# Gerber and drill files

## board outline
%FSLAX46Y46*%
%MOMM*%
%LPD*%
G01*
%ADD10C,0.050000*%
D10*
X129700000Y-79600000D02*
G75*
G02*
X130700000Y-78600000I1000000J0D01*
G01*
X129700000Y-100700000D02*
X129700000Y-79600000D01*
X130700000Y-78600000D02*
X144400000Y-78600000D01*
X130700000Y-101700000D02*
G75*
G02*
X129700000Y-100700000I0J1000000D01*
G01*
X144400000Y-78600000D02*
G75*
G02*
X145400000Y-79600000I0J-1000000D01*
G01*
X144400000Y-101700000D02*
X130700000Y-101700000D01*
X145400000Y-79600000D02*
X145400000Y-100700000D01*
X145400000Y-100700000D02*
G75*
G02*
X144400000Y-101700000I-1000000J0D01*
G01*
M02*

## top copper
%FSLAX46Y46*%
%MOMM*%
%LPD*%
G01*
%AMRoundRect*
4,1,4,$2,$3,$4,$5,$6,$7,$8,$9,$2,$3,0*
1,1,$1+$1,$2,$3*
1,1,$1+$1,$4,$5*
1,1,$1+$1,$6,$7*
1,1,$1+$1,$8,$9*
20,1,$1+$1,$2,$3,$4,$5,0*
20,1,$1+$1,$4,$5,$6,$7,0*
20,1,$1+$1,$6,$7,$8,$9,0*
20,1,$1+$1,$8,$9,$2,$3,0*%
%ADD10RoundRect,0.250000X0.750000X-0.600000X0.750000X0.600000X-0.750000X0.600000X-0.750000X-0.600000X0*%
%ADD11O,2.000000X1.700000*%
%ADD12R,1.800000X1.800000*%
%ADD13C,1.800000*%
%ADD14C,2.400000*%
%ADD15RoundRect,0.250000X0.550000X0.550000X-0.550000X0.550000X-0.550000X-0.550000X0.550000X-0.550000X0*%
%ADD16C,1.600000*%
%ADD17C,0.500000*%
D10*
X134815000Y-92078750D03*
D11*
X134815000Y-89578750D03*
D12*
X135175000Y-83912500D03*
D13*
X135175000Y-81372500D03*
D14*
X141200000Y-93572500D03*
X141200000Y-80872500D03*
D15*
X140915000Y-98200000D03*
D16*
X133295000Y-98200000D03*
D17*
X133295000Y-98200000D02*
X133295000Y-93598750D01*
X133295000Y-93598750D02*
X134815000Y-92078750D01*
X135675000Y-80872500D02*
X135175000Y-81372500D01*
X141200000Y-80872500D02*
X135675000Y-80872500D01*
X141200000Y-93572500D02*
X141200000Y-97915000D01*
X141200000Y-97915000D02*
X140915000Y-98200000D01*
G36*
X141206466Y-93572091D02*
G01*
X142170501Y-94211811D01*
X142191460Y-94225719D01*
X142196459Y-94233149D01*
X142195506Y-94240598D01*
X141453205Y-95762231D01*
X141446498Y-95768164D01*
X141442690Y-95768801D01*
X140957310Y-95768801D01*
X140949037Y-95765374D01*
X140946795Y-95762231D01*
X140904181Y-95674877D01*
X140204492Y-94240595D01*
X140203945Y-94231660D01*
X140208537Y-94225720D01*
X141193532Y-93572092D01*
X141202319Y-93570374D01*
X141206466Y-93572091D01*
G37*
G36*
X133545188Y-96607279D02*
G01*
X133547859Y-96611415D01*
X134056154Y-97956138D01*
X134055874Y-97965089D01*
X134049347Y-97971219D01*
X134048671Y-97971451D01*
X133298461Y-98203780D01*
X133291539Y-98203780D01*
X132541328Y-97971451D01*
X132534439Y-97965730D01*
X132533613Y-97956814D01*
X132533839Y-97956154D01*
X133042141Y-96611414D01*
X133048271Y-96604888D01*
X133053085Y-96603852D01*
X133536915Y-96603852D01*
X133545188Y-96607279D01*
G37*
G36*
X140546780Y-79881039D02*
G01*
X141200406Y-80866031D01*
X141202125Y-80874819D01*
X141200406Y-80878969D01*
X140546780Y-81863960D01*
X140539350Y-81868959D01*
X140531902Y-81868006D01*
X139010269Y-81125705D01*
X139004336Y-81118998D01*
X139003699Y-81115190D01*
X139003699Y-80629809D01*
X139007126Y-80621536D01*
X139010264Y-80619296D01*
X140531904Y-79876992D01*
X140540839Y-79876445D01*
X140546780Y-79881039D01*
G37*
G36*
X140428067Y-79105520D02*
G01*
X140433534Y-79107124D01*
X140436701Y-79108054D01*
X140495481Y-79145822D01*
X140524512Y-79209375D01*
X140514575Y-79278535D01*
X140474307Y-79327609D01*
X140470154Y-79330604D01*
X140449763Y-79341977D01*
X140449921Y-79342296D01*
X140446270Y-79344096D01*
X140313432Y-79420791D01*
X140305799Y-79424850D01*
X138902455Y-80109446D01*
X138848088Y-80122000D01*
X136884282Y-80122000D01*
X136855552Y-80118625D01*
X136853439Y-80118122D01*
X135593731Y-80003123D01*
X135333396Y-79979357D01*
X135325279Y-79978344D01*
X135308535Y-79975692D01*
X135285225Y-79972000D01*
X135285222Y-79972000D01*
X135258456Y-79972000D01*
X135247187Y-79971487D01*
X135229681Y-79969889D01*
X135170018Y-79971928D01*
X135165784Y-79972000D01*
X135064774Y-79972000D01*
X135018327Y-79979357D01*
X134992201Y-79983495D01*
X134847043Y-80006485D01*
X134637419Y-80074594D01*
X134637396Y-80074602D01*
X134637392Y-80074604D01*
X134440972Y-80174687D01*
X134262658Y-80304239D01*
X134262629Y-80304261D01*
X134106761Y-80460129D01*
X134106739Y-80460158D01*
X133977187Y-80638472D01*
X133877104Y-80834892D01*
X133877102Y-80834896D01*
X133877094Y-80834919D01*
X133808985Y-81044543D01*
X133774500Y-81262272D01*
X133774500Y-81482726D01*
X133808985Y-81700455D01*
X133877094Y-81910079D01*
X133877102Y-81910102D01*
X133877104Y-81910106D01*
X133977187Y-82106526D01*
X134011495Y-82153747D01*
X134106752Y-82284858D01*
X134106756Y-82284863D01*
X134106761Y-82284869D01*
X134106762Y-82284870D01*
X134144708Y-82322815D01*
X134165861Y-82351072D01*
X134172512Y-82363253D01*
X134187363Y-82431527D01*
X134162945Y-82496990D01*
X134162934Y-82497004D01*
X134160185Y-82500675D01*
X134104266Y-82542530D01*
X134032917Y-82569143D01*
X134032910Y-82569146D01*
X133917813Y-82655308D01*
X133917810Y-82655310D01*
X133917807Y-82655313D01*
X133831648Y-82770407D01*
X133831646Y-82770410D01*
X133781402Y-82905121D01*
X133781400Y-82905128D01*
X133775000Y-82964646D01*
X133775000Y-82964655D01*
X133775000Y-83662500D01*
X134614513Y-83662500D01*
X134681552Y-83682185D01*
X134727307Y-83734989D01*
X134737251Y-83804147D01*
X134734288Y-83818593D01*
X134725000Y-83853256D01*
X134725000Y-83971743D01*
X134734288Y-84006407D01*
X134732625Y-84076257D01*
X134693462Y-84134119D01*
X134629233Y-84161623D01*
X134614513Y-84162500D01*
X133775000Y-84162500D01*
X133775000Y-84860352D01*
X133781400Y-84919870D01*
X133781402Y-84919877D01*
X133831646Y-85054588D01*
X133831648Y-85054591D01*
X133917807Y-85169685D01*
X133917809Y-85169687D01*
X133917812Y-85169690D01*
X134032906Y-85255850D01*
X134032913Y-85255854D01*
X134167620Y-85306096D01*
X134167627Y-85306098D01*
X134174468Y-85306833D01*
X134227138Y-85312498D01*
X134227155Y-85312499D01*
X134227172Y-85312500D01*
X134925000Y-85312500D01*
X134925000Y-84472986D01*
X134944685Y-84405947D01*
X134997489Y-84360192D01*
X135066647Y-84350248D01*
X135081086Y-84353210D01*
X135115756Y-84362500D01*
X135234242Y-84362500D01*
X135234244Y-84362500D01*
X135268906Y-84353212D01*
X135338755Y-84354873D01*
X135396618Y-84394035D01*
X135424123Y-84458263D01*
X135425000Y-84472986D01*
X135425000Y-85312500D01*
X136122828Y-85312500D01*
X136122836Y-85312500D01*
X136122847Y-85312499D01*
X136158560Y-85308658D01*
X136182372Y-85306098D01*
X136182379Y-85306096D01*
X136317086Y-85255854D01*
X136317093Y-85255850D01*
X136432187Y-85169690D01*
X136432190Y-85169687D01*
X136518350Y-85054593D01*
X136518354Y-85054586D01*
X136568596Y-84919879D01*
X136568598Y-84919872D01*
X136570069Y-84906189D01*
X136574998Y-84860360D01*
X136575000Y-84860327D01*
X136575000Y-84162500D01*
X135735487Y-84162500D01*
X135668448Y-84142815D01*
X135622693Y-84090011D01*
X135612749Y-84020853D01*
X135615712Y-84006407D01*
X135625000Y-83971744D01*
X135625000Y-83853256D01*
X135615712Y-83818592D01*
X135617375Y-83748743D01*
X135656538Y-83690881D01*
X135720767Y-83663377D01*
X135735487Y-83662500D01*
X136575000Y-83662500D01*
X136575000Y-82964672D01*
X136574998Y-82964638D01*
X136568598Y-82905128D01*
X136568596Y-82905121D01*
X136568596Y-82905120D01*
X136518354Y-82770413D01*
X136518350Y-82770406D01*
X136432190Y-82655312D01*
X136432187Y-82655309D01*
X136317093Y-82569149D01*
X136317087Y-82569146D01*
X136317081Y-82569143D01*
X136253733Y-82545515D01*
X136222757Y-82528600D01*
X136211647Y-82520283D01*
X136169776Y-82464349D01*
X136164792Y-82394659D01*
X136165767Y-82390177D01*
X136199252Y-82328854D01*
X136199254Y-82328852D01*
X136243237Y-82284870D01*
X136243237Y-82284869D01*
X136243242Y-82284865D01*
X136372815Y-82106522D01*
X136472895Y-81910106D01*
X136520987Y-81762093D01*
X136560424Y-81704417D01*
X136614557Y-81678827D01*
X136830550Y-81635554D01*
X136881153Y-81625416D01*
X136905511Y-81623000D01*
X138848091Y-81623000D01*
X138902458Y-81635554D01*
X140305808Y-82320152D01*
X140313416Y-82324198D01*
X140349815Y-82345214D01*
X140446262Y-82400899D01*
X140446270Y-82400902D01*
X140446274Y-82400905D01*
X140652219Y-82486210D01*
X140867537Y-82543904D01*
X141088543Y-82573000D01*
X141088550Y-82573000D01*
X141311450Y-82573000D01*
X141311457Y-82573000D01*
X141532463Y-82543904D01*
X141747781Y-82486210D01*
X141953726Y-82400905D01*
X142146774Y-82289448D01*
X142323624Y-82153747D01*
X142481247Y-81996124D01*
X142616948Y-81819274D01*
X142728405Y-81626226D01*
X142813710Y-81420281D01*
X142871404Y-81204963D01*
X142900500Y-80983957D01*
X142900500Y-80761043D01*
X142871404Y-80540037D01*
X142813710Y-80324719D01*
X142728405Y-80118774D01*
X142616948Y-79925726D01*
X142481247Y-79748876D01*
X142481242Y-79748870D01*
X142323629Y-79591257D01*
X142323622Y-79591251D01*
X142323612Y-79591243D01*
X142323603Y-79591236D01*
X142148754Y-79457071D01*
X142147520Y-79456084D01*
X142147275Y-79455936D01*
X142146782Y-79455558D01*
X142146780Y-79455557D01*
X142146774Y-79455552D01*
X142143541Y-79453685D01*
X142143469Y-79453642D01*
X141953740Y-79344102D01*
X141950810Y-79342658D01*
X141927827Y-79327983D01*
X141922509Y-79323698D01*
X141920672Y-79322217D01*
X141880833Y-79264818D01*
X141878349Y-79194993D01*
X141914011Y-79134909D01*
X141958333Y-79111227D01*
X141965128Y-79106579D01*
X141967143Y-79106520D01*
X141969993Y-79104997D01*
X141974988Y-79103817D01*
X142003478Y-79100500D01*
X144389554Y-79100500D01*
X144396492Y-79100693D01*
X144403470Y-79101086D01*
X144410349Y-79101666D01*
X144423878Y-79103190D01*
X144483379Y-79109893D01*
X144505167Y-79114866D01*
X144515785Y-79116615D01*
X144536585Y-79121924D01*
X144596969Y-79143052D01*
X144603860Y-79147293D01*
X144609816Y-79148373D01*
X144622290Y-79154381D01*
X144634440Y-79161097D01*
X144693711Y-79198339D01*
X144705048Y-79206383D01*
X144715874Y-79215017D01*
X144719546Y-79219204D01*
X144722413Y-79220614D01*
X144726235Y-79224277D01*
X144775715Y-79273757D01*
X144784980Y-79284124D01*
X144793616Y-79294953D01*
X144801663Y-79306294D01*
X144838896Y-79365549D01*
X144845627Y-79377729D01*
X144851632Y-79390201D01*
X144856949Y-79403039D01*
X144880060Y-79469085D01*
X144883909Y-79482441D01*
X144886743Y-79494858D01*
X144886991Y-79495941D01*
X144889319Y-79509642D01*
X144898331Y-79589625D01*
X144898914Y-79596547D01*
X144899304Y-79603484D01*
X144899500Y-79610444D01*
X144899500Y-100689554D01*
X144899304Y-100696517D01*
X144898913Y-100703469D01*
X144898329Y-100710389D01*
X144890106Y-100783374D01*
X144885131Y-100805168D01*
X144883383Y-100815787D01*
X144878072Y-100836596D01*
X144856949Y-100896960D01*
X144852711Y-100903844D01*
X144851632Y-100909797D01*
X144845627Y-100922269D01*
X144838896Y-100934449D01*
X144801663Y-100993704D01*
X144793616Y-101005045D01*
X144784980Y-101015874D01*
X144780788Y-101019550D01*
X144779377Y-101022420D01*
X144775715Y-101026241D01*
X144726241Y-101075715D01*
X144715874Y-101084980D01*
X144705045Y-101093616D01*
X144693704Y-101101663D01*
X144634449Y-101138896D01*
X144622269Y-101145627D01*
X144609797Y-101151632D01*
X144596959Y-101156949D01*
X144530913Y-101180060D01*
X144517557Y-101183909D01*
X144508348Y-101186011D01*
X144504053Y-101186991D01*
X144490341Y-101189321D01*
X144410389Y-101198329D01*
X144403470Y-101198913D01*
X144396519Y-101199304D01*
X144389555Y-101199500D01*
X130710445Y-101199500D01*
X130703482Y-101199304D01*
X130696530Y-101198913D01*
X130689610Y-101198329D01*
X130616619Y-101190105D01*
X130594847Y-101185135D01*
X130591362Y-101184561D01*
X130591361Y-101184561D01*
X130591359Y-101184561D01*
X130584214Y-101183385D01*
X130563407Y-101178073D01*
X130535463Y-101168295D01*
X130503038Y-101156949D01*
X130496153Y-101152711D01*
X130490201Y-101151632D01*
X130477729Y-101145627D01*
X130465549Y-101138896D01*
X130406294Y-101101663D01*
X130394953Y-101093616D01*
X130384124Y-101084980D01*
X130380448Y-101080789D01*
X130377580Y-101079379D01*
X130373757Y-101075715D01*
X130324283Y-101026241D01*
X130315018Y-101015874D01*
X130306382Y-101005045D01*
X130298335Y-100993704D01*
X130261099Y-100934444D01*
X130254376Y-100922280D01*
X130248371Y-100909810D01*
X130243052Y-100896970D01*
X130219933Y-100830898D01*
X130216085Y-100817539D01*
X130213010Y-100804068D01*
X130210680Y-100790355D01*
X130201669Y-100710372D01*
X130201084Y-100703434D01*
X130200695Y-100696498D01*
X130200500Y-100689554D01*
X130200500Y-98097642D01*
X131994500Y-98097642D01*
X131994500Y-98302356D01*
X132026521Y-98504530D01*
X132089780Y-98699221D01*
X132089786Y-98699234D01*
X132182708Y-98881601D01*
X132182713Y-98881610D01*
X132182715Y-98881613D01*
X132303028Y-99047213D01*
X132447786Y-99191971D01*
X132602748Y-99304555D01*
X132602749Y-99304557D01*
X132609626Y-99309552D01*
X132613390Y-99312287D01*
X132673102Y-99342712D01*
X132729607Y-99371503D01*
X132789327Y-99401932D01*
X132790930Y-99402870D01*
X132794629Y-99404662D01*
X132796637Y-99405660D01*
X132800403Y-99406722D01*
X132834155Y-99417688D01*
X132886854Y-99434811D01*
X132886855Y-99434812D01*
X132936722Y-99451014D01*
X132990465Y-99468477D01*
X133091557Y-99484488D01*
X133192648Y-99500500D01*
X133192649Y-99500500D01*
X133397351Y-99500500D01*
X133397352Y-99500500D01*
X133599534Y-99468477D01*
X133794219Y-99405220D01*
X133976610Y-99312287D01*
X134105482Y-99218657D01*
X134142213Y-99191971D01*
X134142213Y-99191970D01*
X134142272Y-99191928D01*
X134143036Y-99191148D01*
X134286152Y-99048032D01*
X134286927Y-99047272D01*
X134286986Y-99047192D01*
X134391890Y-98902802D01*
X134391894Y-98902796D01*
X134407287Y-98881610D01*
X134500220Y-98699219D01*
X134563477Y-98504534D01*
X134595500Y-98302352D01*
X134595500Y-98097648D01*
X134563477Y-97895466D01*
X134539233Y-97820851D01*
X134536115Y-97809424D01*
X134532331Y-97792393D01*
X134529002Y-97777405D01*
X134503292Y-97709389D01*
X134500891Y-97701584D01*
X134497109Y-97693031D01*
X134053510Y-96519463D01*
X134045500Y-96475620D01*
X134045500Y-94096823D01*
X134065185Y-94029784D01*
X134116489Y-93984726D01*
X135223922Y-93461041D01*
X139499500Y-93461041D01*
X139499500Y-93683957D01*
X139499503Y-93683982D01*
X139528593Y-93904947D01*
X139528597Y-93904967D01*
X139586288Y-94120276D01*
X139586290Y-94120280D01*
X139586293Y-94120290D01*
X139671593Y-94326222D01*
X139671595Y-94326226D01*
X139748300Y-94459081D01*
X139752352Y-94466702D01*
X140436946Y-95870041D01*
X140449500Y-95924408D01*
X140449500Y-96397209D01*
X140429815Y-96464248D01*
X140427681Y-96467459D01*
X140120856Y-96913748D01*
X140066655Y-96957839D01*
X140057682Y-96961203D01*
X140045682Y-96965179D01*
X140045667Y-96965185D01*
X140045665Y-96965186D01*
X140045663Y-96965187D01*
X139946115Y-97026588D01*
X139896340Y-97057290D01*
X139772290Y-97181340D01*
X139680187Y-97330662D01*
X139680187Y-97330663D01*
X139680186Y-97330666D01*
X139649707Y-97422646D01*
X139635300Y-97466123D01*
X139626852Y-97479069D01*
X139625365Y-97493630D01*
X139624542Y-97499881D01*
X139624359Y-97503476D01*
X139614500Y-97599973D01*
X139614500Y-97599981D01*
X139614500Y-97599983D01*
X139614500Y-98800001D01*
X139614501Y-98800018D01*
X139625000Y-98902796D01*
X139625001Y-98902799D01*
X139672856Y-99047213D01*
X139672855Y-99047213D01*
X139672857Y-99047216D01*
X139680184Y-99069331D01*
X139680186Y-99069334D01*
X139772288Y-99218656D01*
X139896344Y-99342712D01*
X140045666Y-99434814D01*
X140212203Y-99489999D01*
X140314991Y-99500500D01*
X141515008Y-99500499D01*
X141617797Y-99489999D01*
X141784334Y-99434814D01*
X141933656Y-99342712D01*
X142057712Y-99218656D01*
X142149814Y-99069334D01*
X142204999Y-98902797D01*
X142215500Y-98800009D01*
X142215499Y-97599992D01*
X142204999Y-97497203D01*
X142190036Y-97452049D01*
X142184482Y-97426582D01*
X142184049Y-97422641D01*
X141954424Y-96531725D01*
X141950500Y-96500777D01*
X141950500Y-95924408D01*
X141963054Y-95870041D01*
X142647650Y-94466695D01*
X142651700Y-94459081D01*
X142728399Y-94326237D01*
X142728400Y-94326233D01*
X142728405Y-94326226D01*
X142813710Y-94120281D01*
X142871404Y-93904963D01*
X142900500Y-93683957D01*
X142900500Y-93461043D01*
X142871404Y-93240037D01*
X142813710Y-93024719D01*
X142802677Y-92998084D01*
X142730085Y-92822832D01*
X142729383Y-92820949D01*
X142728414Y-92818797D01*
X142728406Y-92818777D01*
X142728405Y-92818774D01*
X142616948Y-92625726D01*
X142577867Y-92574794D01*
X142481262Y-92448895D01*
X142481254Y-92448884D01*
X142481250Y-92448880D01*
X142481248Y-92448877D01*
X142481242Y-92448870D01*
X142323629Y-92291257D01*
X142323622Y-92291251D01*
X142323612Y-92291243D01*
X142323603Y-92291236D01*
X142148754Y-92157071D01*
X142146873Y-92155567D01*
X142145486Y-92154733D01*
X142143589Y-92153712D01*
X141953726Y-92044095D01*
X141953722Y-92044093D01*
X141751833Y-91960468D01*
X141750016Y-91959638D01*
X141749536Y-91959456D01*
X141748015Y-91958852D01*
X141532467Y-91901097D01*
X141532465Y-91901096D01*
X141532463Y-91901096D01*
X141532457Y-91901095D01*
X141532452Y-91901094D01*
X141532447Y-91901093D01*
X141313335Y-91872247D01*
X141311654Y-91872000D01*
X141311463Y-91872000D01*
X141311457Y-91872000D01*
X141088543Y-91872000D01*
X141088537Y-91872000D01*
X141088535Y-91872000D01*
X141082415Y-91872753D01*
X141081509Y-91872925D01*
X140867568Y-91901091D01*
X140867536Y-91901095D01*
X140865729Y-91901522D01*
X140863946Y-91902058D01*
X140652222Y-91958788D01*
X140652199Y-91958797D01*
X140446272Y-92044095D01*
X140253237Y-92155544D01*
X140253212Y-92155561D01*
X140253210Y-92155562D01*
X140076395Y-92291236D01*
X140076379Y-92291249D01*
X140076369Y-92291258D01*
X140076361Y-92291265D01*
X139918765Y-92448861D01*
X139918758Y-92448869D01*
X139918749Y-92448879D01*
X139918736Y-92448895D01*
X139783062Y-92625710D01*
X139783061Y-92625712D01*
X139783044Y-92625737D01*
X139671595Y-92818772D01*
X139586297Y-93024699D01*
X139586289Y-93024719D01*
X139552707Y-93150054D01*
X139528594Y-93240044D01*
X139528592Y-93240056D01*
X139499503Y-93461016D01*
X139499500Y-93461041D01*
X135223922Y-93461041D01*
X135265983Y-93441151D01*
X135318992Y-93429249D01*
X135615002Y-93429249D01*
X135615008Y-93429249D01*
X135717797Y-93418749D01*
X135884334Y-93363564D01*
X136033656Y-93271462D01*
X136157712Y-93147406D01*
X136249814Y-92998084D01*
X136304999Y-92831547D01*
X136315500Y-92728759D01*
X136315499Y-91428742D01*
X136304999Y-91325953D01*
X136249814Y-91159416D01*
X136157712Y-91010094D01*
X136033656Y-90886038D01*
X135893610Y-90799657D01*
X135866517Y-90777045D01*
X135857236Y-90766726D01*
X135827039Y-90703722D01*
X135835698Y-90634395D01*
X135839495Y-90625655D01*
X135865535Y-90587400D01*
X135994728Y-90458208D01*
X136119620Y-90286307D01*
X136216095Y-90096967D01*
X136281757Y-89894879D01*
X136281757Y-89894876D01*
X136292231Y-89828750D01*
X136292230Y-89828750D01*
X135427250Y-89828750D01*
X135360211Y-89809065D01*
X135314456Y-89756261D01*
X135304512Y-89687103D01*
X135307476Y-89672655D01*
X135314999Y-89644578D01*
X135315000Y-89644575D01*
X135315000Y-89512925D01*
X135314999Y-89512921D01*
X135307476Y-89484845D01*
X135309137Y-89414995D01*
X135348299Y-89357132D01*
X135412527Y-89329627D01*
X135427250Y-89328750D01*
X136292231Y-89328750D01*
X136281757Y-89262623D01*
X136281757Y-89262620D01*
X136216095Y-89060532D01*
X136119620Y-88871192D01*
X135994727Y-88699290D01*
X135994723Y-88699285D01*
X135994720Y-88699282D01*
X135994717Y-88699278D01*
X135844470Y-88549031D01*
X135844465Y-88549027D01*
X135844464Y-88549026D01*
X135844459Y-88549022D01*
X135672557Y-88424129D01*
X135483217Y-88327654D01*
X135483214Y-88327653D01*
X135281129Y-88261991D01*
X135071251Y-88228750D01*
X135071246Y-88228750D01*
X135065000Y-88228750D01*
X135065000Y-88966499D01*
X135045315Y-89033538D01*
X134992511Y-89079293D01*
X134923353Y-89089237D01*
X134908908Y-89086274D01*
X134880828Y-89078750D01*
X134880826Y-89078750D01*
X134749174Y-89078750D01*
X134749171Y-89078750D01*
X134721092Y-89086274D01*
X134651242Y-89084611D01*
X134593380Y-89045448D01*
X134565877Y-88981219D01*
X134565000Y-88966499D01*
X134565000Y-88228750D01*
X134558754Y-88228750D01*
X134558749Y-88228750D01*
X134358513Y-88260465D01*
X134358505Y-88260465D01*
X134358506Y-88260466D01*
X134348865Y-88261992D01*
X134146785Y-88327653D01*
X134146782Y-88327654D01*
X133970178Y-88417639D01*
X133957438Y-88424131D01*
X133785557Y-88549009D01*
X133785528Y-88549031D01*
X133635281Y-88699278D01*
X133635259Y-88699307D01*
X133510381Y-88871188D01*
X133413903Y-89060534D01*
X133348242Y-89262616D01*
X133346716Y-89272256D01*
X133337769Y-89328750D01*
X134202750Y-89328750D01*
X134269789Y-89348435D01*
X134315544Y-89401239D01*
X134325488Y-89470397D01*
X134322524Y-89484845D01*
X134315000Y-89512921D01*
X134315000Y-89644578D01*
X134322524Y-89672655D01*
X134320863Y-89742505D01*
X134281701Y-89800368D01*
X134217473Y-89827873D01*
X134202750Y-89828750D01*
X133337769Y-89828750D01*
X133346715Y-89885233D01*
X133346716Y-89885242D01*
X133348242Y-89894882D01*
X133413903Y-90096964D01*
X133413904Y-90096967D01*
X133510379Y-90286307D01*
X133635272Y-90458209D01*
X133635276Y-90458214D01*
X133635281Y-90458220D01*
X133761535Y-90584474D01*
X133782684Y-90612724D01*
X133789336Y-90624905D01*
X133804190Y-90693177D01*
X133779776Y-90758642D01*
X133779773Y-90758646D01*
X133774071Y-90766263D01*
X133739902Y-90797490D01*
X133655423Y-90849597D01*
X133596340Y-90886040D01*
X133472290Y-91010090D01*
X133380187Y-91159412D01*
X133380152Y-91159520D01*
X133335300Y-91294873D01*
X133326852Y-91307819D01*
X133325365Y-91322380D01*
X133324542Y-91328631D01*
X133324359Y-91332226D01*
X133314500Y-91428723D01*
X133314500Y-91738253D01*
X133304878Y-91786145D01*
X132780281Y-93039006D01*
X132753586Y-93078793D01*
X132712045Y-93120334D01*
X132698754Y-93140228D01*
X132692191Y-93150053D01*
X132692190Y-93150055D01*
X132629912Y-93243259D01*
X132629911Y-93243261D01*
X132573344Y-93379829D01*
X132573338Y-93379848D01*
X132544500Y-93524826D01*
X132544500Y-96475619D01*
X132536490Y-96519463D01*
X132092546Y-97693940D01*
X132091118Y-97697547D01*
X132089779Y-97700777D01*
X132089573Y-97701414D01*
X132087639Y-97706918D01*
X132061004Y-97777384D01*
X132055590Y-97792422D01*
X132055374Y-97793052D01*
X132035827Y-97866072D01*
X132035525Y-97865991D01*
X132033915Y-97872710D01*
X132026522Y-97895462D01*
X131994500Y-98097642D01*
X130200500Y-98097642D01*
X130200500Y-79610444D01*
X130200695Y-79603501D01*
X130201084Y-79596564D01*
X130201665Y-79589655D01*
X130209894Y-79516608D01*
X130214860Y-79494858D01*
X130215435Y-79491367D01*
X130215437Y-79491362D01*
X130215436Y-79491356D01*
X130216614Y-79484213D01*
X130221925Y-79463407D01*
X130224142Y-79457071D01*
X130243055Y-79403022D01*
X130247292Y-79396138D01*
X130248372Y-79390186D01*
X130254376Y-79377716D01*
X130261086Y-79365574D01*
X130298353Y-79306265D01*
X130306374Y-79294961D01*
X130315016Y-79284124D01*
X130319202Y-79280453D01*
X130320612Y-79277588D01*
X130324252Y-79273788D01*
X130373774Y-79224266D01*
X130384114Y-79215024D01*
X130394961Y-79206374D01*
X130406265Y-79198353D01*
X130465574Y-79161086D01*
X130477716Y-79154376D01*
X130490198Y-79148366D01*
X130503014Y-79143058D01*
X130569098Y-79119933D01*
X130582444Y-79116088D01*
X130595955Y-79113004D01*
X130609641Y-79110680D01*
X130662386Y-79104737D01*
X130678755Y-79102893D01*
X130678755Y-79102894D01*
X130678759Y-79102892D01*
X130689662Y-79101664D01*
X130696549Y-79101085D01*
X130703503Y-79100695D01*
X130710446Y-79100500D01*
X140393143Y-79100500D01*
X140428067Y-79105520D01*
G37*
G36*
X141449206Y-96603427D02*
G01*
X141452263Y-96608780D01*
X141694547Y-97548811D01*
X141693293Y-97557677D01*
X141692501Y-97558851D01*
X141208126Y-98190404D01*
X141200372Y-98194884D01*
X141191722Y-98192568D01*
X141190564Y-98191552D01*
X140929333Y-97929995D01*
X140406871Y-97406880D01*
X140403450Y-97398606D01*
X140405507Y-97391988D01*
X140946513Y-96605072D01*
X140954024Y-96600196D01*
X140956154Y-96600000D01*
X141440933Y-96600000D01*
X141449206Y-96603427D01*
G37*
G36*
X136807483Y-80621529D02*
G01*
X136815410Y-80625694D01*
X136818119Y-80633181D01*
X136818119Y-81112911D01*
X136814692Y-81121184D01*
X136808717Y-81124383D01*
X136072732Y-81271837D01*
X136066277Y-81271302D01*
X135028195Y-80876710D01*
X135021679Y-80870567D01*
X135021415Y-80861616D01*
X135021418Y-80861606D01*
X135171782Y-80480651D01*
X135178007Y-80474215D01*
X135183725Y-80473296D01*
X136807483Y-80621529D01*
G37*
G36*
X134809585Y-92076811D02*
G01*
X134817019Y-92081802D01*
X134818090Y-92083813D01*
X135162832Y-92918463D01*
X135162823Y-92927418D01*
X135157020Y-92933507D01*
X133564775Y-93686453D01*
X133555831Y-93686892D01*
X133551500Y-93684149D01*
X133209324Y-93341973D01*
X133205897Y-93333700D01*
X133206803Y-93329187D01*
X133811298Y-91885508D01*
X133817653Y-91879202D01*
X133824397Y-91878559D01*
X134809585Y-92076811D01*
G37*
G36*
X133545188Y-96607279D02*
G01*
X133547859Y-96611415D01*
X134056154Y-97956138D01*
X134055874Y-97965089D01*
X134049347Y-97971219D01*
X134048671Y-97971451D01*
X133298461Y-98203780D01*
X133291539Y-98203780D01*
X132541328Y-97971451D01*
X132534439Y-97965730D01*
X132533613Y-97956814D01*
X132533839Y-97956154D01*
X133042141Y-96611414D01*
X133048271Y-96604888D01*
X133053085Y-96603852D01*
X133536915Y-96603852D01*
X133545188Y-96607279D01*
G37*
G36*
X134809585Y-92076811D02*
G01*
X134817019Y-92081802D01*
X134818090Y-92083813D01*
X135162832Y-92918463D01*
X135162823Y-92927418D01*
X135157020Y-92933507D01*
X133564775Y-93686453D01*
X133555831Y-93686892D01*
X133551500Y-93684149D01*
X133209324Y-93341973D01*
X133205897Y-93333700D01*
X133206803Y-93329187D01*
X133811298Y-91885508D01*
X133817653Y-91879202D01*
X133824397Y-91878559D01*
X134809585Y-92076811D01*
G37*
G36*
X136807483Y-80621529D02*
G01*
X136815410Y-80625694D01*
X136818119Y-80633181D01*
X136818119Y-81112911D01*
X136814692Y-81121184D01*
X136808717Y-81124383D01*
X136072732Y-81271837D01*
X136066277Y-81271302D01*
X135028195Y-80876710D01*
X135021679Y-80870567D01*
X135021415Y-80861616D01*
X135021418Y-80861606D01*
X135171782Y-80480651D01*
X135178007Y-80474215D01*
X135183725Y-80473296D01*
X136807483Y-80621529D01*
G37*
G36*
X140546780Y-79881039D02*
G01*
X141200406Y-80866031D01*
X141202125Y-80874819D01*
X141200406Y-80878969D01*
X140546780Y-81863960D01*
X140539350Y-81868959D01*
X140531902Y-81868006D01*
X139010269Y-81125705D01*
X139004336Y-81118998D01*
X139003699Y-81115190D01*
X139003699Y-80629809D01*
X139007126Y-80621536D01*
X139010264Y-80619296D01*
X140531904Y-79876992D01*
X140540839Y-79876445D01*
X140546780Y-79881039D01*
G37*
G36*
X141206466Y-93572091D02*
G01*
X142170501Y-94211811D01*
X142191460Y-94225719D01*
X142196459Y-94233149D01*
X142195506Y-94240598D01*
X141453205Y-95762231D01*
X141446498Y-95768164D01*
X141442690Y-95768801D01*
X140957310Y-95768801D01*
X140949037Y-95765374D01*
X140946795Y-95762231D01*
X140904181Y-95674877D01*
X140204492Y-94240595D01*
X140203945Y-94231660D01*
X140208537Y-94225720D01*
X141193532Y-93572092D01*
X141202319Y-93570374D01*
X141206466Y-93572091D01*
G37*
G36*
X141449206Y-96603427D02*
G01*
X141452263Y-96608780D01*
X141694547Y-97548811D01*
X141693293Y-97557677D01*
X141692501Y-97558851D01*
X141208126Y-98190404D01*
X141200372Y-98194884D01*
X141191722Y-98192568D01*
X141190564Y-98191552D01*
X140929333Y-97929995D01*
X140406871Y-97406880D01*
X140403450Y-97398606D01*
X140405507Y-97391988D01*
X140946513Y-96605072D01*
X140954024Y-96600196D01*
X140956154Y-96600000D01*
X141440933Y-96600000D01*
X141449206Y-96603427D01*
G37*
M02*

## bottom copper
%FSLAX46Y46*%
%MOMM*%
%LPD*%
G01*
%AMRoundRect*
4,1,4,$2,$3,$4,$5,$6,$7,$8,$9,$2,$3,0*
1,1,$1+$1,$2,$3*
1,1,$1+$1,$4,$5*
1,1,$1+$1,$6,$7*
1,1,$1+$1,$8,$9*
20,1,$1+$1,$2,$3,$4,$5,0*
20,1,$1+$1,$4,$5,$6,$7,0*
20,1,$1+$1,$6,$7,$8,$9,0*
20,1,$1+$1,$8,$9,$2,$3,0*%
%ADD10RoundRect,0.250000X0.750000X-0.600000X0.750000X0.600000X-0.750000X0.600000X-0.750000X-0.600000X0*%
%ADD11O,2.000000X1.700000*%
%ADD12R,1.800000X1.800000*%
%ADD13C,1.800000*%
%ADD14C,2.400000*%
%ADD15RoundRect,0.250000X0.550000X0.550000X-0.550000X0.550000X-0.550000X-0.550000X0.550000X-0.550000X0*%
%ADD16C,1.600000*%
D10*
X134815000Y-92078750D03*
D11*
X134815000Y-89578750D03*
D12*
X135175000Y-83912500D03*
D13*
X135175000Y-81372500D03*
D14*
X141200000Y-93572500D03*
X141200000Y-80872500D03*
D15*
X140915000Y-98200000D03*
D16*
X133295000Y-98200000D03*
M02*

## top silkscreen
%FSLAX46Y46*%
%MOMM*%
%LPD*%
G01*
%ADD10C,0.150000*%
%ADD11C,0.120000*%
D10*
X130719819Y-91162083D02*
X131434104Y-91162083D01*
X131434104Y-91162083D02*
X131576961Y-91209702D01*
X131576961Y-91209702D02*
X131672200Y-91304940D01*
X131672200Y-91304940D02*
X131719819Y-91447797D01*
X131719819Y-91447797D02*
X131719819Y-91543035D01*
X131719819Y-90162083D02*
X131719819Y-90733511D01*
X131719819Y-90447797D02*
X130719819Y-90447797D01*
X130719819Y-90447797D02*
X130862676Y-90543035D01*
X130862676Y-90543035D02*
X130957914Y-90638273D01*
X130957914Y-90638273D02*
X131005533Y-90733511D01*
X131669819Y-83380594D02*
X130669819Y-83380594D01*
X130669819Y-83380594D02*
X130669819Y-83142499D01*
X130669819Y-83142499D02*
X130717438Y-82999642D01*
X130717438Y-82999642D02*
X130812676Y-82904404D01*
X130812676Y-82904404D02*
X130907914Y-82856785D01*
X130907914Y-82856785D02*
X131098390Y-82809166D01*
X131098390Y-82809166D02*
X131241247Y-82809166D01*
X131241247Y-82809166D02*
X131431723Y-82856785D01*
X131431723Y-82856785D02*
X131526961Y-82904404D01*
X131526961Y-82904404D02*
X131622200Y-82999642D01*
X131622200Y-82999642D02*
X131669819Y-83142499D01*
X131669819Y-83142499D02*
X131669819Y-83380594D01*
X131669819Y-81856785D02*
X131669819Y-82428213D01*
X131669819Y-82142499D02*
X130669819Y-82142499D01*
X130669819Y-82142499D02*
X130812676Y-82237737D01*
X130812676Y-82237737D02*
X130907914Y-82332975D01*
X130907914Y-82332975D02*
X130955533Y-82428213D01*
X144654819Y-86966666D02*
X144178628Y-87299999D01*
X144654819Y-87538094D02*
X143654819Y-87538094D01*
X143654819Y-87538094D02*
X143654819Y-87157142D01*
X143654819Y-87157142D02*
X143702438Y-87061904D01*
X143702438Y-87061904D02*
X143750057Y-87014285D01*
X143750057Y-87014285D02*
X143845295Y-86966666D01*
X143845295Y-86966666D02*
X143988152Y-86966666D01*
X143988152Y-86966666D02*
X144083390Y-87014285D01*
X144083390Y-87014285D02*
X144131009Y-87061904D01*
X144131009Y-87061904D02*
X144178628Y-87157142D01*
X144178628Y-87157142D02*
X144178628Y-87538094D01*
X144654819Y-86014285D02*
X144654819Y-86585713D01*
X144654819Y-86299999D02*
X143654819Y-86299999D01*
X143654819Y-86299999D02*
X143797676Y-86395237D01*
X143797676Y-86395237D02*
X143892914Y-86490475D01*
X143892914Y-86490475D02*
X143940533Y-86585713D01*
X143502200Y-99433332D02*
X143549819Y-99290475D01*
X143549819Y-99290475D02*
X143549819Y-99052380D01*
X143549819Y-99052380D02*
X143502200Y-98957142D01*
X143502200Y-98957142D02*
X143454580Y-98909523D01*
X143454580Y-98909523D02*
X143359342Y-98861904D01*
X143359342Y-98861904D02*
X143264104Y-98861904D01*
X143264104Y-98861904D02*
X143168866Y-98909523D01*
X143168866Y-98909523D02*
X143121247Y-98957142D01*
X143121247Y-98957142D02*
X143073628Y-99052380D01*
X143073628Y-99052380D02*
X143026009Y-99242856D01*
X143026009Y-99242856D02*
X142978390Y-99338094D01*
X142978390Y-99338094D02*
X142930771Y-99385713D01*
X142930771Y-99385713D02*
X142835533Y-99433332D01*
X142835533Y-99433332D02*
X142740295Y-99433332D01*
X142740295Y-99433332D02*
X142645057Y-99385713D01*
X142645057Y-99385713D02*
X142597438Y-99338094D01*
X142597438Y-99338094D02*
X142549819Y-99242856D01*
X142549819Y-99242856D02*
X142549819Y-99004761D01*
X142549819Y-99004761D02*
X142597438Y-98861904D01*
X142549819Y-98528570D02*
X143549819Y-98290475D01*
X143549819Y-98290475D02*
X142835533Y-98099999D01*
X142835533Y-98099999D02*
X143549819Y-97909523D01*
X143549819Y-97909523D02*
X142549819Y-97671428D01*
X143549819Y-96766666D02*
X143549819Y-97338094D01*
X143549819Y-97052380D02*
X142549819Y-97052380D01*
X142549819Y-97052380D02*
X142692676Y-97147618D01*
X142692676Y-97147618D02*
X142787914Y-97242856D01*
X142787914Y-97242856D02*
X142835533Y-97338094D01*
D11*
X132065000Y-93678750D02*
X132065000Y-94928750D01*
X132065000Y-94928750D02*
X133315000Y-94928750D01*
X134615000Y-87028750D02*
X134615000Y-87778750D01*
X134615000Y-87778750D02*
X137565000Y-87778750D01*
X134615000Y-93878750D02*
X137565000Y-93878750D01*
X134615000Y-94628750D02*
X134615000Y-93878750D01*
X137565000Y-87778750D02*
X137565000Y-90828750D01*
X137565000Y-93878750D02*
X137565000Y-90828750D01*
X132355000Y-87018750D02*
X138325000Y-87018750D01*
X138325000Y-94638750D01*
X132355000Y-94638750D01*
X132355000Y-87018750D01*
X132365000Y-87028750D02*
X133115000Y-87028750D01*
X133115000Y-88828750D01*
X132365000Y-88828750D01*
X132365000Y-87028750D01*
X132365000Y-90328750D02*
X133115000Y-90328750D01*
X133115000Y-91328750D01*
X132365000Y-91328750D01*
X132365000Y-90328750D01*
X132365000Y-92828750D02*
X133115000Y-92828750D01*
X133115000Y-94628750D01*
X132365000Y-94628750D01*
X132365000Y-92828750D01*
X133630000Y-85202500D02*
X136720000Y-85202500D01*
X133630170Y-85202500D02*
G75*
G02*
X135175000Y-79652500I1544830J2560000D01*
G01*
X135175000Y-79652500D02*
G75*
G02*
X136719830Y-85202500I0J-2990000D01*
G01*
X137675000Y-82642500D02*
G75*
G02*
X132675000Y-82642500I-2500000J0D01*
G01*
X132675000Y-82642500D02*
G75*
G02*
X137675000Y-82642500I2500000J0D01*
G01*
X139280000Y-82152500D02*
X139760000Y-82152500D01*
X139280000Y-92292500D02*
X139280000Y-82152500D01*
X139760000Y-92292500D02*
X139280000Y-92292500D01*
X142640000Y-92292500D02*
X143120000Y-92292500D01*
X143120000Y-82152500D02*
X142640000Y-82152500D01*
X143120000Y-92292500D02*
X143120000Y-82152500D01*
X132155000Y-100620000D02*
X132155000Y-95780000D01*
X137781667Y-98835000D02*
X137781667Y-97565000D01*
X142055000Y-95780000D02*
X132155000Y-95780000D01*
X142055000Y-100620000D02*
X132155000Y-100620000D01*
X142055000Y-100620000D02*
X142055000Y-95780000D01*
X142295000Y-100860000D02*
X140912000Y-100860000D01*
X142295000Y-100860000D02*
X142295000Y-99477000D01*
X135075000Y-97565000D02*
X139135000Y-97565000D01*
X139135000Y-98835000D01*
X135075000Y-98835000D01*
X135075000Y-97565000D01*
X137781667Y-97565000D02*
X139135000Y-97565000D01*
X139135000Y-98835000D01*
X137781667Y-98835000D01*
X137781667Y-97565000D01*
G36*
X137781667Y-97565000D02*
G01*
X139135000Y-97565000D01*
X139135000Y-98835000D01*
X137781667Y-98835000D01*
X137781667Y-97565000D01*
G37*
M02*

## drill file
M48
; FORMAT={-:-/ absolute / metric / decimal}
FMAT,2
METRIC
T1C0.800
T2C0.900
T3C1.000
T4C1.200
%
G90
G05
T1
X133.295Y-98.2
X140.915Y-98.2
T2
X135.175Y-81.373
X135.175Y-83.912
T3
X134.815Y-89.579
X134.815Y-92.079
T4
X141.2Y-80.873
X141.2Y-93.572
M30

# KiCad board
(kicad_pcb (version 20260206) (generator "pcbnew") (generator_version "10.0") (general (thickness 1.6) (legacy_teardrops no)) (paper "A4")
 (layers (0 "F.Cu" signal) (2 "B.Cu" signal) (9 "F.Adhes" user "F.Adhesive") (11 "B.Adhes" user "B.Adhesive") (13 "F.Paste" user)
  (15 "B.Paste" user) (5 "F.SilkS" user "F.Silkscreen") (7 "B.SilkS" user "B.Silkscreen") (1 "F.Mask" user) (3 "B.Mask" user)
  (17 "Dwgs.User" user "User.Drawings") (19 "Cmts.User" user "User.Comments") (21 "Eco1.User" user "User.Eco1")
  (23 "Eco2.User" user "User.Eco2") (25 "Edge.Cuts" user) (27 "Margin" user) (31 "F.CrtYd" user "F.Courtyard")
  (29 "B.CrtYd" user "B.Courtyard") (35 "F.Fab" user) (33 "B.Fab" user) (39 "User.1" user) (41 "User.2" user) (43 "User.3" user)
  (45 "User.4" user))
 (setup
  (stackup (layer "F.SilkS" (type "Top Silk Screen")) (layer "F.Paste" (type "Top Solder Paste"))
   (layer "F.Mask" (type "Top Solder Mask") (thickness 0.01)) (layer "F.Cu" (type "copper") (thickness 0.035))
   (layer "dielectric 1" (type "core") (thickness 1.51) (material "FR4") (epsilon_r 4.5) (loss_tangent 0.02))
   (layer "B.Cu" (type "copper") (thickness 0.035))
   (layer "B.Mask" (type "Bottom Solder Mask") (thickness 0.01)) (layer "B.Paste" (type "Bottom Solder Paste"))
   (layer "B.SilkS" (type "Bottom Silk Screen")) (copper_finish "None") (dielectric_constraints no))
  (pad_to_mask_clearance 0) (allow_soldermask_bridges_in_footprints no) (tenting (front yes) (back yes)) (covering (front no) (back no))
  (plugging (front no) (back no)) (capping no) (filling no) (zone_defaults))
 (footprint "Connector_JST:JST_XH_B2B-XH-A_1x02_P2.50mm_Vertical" (layer "F.Cu") (at 134.815 92.07875 90)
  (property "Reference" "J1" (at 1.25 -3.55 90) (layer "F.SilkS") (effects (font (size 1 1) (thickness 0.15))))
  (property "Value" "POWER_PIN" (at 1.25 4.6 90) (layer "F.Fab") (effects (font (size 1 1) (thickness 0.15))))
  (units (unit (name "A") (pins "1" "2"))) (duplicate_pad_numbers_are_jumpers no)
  (fp_line (start -1.6 -2.75) (end -2.85 -2.75) (stroke (width 0.12) (type solid)) (layer "F.SilkS"))
  (fp_line (start -2.85 -2.75) (end -2.85 -1.5) (stroke (width 0.12) (type solid)) (layer "F.SilkS"))
  (fp_line (start 5.05 -0.2) (end 4.3 -0.2) (stroke (width 0.12) (type solid)) (layer "F.SilkS"))
  (fp_line (start 4.3 -0.2) (end 4.3 2.75) (stroke (width 0.12) (type solid)) (layer "F.SilkS"))
  (fp_line (start -1.8 -0.2) (end -1.8 2.75) (stroke (width 0.12) (type solid)) (layer "F.SilkS"))
  (fp_line (start -2.55 -0.2) (end -1.8 -0.2) (stroke (width 0.12) (type solid)) (layer "F.SilkS"))
  (fp_line (start 4.3 2.75) (end 1.25 2.75) (stroke (width 0.12) (type solid)) (layer "F.SilkS"))
  (fp_line (start -1.8 2.75) (end 1.25 2.75) (stroke (width 0.12) (type solid)) (layer "F.SilkS"))
  (fp_rect (start -2.56 -2.46) (end 5.06 3.51) (stroke (width 0.12) (type solid)) (fill no) (layer "F.SilkS"))
  (fp_rect (start 3.25 -2.45) (end 5.05 -1.7) (stroke (width 0.12) (type solid)) (fill no) (layer "F.SilkS"))
  (fp_rect (start 0.75 -2.45) (end 1.75 -1.7) (stroke (width 0.12) (type solid)) (fill no) (layer "F.SilkS"))
  (fp_rect (start -2.55 -2.45) (end -0.75 -1.7) (stroke (width 0.12) (type solid)) (fill no) (layer "F.SilkS"))
  (pad "1" thru_hole roundrect (at 0 0 90) (size 1.7 2) (drill 1) (layers "*.Cu" "*.Mask") (remove_unused_layers no)
   (roundrect_rratio 0.147059) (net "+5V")
   (teardrops (best_length_ratio 0.5) (max_length 1) (best_width_ratio 1) (max_width 2) (curved_edges no) (filter_ratio 0.9) (enabled yes)
    (allow_two_segments yes) (prefer_zone_connections yes)))
  (pad "2" thru_hole oval (at 2.5 0 90) (size 1.7 2) (drill 1) (layers "*.Cu" "*.Mask") (remove_unused_layers no) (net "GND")
   (teardrops (best_length_ratio 0.5) (max_length 1) (best_width_ratio 1) (max_width 2) (curved_edges no) (filter_ratio 0.9) (enabled yes)
    (allow_two_segments yes) (prefer_zone_connections yes))))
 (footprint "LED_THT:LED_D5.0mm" (layer "F.Cu") (at 135.175 83.9125 90)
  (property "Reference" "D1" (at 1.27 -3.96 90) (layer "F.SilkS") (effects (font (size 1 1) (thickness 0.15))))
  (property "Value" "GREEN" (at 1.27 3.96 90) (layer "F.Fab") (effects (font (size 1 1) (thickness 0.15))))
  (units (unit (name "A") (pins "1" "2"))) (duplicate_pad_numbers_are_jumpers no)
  (fp_line (start -1.29 -1.545) (end -1.29 1.545) (stroke (width 0.12) (type solid)) (layer "F.SilkS"))
  (fp_arc (start -1.29 -1.54483) (mid 2.071779 -2.880495) (end 4.26 0) (stroke (width 0.12) (type solid)) (layer "F.SilkS"))
  (fp_arc (start 4.26 0) (mid 2.071779 2.880495) (end -1.29 1.54483) (stroke (width 0.12) (type solid)) (layer "F.SilkS"))
  (fp_circle (center 1.27 0) (end 3.77 0) (stroke (width 0.12) (type solid)) (fill no) (layer "F.SilkS"))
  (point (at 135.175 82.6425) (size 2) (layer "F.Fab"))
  (pad "1" thru_hole rect (at 0 0 90) (size 1.8 1.8) (drill 0.9) (layers "*.Cu" "*.Mask") (remove_unused_layers no) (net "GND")
   (teardrops (best_length_ratio 0.5) (max_length 1) (best_width_ratio 1) (max_width 2) (curved_edges no) (filter_ratio 0.9) (enabled yes)
    (allow_two_segments yes) (prefer_zone_connections yes)))
  (pad "2" thru_hole circle (at 2.54 0 90) (size 1.8 1.8) (drill 0.9) (layers "*.Cu" "*.Mask") (remove_unused_layers no) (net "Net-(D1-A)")
   (teardrops (best_length_ratio 0.5) (max_length 1) (best_width_ratio 1) (max_width 2) (curved_edges no) (filter_ratio 0.9) (enabled yes)
    (allow_two_segments yes) (prefer_zone_connections yes))))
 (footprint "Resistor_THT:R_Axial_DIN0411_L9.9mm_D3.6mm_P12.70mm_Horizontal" (layer "F.Cu") (at 141.2 93.5725 90)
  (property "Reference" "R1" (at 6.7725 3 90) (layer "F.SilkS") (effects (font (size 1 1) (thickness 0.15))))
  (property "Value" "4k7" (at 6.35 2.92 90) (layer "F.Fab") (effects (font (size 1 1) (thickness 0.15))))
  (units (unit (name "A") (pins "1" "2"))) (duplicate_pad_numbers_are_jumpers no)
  (fp_line (start 11.42 -1.92) (end 11.42 -1.44) (stroke (width 0.12) (type solid)) (layer "F.SilkS"))
  (fp_line (start 1.28 -1.92) (end 11.42 -1.92) (stroke (width 0.12) (type solid)) (layer "F.SilkS"))
  (fp_line (start 1.28 -1.44) (end 1.28 -1.92) (stroke (width 0.12) (type solid)) (layer "F.SilkS"))
  (fp_line (start 1.28 1.44) (end 1.28 1.92) (stroke (width 0.12) (type solid)) (layer "F.SilkS"))
  (fp_line (start 11.42 1.92) (end 11.42 1.44) (stroke (width 0.12) (type solid)) (layer "F.SilkS"))
  (fp_line (start 1.28 1.92) (end 11.42 1.92) (stroke (width 0.12) (type solid)) (layer "F.SilkS"))
  (pad "1" thru_hole circle (at 0 0 90) (size 2.4 2.4) (drill 1.2) (layers "*.Cu" "*.Mask") (remove_unused_layers no) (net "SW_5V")
   (teardrops (best_length_ratio 0.5) (max_length 1) (best_width_ratio 1) (max_width 2) (curved_edges no) (filter_ratio 0.9) (enabled yes)
    (allow_two_segments yes) (prefer_zone_connections yes)))
  (pad "2" thru_hole circle (at 12.7 0 90) (size 2.4 2.4) (drill 1.2) (layers "*.Cu" "*.Mask") (remove_unused_layers no) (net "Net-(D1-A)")
   (teardrops (best_length_ratio 0.5) (max_length 1) (best_width_ratio 1) (max_width 2) (curved_edges no) (filter_ratio 0.9) (enabled yes)
    (allow_two_segments yes) (prefer_zone_connections yes))))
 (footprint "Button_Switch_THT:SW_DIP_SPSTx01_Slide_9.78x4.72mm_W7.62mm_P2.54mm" (layer "F.Cu") (at 140.915 98.2 180)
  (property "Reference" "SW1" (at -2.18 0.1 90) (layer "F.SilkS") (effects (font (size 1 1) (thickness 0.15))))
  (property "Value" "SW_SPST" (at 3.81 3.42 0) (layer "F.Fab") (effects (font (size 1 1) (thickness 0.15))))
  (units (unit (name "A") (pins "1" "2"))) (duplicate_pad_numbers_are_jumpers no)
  (fp_line (start 8.76 -2.42) (end 8.76 2.42) (stroke (width 0.12) (type solid)) (layer "F.SilkS"))
  (fp_line (start 3.133333 -0.635) (end 3.133333 0.635) (stroke (width 0.12) (type solid)) (layer "F.SilkS"))
  (fp_line (start -1.14 2.42) (end 8.76 2.42) (stroke (width 0.12) (type solid)) (layer "F.SilkS"))
  (fp_line (start -1.14 -2.42) (end 8.76 -2.42) (stroke (width 0.12) (type solid)) (layer "F.SilkS"))
  (fp_line (start -1.14 -2.42) (end -1.14 2.42) (stroke (width 0.12) (type solid)) (layer "F.SilkS"))
  (fp_line (start -1.38 -2.66) (end 0.003 -2.66) (stroke (width 0.12) (type solid)) (layer "F.SilkS"))
  (fp_line (start -1.38 -2.66) (end -1.38 -1.277) (stroke (width 0.12) (type solid)) (layer "F.SilkS"))
  (fp_rect (start 1.78 -0.635) (end 5.84 0.635) (stroke (width 0.12) (type solid)) (fill no) (layer "F.SilkS"))
  (fp_rect (start 1.78 -0.635) (end 3.133333 0.635) (stroke (width 0.12) (type solid)) (fill yes) (layer "F.SilkS"))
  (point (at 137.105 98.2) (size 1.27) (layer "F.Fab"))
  (pad "1" thru_hole roundrect (at 0 0 180) (size 1.6 1.6) (drill 0.8) (layers "*.Cu" "*.Mask") (remove_unused_layers no)
   (roundrect_rratio 0.15625) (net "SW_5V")
   (teardrops (best_length_ratio 0.5) (max_length 1) (best_width_ratio 1) (max_width 2) (curved_edges no) (filter_ratio 0.9) (enabled yes)
    (allow_two_segments yes) (prefer_zone_connections yes)))
  (pad "2" thru_hole circle (at 7.62 0 180) (size 1.6 1.6) (drill 0.8) (layers "*.Cu" "*.Mask") (remove_unused_layers no) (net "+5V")
   (teardrops (best_length_ratio 0.5) (max_length 1) (best_width_ratio 1) (max_width 2) (curved_edges no) (filter_ratio 0.9) (enabled yes)
    (allow_two_segments yes) (prefer_zone_connections yes))))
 (gr_arc (start 129.7 79.6) (mid 129.992893 78.892893) (end 130.7 78.6) (stroke (width 0.05) (type default)) (layer "Edge.Cuts"))
 (gr_line (start 129.7 100.7) (end 129.7 79.6) (stroke (width 0.05) (type default)) (layer "Edge.Cuts"))
 (gr_line (start 130.7 78.6) (end 144.4 78.6) (stroke (width 0.05) (type default)) (layer "Edge.Cuts"))
 (gr_arc (start 130.7 101.7) (mid 129.992893 101.407107) (end 129.7 100.7) (stroke (width 0.05) (type default)) (layer "Edge.Cuts"))
 (gr_arc (start 144.4 78.6) (mid 145.107107 78.892893) (end 145.4 79.6) (stroke (width 0.05) (type default)) (layer "Edge.Cuts"))
 (gr_line (start 144.4 101.7) (end 130.7 101.7) (stroke (width 0.05) (type default)) (layer "Edge.Cuts"))
 (gr_line (start 145.4 79.6) (end 145.4 100.7) (stroke (width 0.05) (type default)) (layer "Edge.Cuts"))
 (gr_arc (start 145.4 100.7) (mid 145.107107 101.407107) (end 144.4 101.7) (stroke (width 0.05) (type default)) (layer "Edge.Cuts"))
 (segment (start 133.295 98.2) (end 133.295 93.59875) (width 0.5) (layer "F.Cu") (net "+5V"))
 (segment (start 133.295 93.59875) (end 134.815 92.07875) (width 0.5) (layer "F.Cu") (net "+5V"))
 (segment (start 135.675 80.8725) (end 135.175 81.3725) (width 0.5) (layer "F.Cu") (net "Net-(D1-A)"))
 (segment (start 141.2 80.8725) (end 135.675 80.8725) (width 0.5) (layer "F.Cu") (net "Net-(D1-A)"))
 (segment (start 141.2 93.5725) (end 141.2 97.915) (width 0.5) (layer "F.Cu") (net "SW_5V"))
 (segment (start 141.2 97.915) (end 140.915 98.2) (width 0.5) (layer "F.Cu") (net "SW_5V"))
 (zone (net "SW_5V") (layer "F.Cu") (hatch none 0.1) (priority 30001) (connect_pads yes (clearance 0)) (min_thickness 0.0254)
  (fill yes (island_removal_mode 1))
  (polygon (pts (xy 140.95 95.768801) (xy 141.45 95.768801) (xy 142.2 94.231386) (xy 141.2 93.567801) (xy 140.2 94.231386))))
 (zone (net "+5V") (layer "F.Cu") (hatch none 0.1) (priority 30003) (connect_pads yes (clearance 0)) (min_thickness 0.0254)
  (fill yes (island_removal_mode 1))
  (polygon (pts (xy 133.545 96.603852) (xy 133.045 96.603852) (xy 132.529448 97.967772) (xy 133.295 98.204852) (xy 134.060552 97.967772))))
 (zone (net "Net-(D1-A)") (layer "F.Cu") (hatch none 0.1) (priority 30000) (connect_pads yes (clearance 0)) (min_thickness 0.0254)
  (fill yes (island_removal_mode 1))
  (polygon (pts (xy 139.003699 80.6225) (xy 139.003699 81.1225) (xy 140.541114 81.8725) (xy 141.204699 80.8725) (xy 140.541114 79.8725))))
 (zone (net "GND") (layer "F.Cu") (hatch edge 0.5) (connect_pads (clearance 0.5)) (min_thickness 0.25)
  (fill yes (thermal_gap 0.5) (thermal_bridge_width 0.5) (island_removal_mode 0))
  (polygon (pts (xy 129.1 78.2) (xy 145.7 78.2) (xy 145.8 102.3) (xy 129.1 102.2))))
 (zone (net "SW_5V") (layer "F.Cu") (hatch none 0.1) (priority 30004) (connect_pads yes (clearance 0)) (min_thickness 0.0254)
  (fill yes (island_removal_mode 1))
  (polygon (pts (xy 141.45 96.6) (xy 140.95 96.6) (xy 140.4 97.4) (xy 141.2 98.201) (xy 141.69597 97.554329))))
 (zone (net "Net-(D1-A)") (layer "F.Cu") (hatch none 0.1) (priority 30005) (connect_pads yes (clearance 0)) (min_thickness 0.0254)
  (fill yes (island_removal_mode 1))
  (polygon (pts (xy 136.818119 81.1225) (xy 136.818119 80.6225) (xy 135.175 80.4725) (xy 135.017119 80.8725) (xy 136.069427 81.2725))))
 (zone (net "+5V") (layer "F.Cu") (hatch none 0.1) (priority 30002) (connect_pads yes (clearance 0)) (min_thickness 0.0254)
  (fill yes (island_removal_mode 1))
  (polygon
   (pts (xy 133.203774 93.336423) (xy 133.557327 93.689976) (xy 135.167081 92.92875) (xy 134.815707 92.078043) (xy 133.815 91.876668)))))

